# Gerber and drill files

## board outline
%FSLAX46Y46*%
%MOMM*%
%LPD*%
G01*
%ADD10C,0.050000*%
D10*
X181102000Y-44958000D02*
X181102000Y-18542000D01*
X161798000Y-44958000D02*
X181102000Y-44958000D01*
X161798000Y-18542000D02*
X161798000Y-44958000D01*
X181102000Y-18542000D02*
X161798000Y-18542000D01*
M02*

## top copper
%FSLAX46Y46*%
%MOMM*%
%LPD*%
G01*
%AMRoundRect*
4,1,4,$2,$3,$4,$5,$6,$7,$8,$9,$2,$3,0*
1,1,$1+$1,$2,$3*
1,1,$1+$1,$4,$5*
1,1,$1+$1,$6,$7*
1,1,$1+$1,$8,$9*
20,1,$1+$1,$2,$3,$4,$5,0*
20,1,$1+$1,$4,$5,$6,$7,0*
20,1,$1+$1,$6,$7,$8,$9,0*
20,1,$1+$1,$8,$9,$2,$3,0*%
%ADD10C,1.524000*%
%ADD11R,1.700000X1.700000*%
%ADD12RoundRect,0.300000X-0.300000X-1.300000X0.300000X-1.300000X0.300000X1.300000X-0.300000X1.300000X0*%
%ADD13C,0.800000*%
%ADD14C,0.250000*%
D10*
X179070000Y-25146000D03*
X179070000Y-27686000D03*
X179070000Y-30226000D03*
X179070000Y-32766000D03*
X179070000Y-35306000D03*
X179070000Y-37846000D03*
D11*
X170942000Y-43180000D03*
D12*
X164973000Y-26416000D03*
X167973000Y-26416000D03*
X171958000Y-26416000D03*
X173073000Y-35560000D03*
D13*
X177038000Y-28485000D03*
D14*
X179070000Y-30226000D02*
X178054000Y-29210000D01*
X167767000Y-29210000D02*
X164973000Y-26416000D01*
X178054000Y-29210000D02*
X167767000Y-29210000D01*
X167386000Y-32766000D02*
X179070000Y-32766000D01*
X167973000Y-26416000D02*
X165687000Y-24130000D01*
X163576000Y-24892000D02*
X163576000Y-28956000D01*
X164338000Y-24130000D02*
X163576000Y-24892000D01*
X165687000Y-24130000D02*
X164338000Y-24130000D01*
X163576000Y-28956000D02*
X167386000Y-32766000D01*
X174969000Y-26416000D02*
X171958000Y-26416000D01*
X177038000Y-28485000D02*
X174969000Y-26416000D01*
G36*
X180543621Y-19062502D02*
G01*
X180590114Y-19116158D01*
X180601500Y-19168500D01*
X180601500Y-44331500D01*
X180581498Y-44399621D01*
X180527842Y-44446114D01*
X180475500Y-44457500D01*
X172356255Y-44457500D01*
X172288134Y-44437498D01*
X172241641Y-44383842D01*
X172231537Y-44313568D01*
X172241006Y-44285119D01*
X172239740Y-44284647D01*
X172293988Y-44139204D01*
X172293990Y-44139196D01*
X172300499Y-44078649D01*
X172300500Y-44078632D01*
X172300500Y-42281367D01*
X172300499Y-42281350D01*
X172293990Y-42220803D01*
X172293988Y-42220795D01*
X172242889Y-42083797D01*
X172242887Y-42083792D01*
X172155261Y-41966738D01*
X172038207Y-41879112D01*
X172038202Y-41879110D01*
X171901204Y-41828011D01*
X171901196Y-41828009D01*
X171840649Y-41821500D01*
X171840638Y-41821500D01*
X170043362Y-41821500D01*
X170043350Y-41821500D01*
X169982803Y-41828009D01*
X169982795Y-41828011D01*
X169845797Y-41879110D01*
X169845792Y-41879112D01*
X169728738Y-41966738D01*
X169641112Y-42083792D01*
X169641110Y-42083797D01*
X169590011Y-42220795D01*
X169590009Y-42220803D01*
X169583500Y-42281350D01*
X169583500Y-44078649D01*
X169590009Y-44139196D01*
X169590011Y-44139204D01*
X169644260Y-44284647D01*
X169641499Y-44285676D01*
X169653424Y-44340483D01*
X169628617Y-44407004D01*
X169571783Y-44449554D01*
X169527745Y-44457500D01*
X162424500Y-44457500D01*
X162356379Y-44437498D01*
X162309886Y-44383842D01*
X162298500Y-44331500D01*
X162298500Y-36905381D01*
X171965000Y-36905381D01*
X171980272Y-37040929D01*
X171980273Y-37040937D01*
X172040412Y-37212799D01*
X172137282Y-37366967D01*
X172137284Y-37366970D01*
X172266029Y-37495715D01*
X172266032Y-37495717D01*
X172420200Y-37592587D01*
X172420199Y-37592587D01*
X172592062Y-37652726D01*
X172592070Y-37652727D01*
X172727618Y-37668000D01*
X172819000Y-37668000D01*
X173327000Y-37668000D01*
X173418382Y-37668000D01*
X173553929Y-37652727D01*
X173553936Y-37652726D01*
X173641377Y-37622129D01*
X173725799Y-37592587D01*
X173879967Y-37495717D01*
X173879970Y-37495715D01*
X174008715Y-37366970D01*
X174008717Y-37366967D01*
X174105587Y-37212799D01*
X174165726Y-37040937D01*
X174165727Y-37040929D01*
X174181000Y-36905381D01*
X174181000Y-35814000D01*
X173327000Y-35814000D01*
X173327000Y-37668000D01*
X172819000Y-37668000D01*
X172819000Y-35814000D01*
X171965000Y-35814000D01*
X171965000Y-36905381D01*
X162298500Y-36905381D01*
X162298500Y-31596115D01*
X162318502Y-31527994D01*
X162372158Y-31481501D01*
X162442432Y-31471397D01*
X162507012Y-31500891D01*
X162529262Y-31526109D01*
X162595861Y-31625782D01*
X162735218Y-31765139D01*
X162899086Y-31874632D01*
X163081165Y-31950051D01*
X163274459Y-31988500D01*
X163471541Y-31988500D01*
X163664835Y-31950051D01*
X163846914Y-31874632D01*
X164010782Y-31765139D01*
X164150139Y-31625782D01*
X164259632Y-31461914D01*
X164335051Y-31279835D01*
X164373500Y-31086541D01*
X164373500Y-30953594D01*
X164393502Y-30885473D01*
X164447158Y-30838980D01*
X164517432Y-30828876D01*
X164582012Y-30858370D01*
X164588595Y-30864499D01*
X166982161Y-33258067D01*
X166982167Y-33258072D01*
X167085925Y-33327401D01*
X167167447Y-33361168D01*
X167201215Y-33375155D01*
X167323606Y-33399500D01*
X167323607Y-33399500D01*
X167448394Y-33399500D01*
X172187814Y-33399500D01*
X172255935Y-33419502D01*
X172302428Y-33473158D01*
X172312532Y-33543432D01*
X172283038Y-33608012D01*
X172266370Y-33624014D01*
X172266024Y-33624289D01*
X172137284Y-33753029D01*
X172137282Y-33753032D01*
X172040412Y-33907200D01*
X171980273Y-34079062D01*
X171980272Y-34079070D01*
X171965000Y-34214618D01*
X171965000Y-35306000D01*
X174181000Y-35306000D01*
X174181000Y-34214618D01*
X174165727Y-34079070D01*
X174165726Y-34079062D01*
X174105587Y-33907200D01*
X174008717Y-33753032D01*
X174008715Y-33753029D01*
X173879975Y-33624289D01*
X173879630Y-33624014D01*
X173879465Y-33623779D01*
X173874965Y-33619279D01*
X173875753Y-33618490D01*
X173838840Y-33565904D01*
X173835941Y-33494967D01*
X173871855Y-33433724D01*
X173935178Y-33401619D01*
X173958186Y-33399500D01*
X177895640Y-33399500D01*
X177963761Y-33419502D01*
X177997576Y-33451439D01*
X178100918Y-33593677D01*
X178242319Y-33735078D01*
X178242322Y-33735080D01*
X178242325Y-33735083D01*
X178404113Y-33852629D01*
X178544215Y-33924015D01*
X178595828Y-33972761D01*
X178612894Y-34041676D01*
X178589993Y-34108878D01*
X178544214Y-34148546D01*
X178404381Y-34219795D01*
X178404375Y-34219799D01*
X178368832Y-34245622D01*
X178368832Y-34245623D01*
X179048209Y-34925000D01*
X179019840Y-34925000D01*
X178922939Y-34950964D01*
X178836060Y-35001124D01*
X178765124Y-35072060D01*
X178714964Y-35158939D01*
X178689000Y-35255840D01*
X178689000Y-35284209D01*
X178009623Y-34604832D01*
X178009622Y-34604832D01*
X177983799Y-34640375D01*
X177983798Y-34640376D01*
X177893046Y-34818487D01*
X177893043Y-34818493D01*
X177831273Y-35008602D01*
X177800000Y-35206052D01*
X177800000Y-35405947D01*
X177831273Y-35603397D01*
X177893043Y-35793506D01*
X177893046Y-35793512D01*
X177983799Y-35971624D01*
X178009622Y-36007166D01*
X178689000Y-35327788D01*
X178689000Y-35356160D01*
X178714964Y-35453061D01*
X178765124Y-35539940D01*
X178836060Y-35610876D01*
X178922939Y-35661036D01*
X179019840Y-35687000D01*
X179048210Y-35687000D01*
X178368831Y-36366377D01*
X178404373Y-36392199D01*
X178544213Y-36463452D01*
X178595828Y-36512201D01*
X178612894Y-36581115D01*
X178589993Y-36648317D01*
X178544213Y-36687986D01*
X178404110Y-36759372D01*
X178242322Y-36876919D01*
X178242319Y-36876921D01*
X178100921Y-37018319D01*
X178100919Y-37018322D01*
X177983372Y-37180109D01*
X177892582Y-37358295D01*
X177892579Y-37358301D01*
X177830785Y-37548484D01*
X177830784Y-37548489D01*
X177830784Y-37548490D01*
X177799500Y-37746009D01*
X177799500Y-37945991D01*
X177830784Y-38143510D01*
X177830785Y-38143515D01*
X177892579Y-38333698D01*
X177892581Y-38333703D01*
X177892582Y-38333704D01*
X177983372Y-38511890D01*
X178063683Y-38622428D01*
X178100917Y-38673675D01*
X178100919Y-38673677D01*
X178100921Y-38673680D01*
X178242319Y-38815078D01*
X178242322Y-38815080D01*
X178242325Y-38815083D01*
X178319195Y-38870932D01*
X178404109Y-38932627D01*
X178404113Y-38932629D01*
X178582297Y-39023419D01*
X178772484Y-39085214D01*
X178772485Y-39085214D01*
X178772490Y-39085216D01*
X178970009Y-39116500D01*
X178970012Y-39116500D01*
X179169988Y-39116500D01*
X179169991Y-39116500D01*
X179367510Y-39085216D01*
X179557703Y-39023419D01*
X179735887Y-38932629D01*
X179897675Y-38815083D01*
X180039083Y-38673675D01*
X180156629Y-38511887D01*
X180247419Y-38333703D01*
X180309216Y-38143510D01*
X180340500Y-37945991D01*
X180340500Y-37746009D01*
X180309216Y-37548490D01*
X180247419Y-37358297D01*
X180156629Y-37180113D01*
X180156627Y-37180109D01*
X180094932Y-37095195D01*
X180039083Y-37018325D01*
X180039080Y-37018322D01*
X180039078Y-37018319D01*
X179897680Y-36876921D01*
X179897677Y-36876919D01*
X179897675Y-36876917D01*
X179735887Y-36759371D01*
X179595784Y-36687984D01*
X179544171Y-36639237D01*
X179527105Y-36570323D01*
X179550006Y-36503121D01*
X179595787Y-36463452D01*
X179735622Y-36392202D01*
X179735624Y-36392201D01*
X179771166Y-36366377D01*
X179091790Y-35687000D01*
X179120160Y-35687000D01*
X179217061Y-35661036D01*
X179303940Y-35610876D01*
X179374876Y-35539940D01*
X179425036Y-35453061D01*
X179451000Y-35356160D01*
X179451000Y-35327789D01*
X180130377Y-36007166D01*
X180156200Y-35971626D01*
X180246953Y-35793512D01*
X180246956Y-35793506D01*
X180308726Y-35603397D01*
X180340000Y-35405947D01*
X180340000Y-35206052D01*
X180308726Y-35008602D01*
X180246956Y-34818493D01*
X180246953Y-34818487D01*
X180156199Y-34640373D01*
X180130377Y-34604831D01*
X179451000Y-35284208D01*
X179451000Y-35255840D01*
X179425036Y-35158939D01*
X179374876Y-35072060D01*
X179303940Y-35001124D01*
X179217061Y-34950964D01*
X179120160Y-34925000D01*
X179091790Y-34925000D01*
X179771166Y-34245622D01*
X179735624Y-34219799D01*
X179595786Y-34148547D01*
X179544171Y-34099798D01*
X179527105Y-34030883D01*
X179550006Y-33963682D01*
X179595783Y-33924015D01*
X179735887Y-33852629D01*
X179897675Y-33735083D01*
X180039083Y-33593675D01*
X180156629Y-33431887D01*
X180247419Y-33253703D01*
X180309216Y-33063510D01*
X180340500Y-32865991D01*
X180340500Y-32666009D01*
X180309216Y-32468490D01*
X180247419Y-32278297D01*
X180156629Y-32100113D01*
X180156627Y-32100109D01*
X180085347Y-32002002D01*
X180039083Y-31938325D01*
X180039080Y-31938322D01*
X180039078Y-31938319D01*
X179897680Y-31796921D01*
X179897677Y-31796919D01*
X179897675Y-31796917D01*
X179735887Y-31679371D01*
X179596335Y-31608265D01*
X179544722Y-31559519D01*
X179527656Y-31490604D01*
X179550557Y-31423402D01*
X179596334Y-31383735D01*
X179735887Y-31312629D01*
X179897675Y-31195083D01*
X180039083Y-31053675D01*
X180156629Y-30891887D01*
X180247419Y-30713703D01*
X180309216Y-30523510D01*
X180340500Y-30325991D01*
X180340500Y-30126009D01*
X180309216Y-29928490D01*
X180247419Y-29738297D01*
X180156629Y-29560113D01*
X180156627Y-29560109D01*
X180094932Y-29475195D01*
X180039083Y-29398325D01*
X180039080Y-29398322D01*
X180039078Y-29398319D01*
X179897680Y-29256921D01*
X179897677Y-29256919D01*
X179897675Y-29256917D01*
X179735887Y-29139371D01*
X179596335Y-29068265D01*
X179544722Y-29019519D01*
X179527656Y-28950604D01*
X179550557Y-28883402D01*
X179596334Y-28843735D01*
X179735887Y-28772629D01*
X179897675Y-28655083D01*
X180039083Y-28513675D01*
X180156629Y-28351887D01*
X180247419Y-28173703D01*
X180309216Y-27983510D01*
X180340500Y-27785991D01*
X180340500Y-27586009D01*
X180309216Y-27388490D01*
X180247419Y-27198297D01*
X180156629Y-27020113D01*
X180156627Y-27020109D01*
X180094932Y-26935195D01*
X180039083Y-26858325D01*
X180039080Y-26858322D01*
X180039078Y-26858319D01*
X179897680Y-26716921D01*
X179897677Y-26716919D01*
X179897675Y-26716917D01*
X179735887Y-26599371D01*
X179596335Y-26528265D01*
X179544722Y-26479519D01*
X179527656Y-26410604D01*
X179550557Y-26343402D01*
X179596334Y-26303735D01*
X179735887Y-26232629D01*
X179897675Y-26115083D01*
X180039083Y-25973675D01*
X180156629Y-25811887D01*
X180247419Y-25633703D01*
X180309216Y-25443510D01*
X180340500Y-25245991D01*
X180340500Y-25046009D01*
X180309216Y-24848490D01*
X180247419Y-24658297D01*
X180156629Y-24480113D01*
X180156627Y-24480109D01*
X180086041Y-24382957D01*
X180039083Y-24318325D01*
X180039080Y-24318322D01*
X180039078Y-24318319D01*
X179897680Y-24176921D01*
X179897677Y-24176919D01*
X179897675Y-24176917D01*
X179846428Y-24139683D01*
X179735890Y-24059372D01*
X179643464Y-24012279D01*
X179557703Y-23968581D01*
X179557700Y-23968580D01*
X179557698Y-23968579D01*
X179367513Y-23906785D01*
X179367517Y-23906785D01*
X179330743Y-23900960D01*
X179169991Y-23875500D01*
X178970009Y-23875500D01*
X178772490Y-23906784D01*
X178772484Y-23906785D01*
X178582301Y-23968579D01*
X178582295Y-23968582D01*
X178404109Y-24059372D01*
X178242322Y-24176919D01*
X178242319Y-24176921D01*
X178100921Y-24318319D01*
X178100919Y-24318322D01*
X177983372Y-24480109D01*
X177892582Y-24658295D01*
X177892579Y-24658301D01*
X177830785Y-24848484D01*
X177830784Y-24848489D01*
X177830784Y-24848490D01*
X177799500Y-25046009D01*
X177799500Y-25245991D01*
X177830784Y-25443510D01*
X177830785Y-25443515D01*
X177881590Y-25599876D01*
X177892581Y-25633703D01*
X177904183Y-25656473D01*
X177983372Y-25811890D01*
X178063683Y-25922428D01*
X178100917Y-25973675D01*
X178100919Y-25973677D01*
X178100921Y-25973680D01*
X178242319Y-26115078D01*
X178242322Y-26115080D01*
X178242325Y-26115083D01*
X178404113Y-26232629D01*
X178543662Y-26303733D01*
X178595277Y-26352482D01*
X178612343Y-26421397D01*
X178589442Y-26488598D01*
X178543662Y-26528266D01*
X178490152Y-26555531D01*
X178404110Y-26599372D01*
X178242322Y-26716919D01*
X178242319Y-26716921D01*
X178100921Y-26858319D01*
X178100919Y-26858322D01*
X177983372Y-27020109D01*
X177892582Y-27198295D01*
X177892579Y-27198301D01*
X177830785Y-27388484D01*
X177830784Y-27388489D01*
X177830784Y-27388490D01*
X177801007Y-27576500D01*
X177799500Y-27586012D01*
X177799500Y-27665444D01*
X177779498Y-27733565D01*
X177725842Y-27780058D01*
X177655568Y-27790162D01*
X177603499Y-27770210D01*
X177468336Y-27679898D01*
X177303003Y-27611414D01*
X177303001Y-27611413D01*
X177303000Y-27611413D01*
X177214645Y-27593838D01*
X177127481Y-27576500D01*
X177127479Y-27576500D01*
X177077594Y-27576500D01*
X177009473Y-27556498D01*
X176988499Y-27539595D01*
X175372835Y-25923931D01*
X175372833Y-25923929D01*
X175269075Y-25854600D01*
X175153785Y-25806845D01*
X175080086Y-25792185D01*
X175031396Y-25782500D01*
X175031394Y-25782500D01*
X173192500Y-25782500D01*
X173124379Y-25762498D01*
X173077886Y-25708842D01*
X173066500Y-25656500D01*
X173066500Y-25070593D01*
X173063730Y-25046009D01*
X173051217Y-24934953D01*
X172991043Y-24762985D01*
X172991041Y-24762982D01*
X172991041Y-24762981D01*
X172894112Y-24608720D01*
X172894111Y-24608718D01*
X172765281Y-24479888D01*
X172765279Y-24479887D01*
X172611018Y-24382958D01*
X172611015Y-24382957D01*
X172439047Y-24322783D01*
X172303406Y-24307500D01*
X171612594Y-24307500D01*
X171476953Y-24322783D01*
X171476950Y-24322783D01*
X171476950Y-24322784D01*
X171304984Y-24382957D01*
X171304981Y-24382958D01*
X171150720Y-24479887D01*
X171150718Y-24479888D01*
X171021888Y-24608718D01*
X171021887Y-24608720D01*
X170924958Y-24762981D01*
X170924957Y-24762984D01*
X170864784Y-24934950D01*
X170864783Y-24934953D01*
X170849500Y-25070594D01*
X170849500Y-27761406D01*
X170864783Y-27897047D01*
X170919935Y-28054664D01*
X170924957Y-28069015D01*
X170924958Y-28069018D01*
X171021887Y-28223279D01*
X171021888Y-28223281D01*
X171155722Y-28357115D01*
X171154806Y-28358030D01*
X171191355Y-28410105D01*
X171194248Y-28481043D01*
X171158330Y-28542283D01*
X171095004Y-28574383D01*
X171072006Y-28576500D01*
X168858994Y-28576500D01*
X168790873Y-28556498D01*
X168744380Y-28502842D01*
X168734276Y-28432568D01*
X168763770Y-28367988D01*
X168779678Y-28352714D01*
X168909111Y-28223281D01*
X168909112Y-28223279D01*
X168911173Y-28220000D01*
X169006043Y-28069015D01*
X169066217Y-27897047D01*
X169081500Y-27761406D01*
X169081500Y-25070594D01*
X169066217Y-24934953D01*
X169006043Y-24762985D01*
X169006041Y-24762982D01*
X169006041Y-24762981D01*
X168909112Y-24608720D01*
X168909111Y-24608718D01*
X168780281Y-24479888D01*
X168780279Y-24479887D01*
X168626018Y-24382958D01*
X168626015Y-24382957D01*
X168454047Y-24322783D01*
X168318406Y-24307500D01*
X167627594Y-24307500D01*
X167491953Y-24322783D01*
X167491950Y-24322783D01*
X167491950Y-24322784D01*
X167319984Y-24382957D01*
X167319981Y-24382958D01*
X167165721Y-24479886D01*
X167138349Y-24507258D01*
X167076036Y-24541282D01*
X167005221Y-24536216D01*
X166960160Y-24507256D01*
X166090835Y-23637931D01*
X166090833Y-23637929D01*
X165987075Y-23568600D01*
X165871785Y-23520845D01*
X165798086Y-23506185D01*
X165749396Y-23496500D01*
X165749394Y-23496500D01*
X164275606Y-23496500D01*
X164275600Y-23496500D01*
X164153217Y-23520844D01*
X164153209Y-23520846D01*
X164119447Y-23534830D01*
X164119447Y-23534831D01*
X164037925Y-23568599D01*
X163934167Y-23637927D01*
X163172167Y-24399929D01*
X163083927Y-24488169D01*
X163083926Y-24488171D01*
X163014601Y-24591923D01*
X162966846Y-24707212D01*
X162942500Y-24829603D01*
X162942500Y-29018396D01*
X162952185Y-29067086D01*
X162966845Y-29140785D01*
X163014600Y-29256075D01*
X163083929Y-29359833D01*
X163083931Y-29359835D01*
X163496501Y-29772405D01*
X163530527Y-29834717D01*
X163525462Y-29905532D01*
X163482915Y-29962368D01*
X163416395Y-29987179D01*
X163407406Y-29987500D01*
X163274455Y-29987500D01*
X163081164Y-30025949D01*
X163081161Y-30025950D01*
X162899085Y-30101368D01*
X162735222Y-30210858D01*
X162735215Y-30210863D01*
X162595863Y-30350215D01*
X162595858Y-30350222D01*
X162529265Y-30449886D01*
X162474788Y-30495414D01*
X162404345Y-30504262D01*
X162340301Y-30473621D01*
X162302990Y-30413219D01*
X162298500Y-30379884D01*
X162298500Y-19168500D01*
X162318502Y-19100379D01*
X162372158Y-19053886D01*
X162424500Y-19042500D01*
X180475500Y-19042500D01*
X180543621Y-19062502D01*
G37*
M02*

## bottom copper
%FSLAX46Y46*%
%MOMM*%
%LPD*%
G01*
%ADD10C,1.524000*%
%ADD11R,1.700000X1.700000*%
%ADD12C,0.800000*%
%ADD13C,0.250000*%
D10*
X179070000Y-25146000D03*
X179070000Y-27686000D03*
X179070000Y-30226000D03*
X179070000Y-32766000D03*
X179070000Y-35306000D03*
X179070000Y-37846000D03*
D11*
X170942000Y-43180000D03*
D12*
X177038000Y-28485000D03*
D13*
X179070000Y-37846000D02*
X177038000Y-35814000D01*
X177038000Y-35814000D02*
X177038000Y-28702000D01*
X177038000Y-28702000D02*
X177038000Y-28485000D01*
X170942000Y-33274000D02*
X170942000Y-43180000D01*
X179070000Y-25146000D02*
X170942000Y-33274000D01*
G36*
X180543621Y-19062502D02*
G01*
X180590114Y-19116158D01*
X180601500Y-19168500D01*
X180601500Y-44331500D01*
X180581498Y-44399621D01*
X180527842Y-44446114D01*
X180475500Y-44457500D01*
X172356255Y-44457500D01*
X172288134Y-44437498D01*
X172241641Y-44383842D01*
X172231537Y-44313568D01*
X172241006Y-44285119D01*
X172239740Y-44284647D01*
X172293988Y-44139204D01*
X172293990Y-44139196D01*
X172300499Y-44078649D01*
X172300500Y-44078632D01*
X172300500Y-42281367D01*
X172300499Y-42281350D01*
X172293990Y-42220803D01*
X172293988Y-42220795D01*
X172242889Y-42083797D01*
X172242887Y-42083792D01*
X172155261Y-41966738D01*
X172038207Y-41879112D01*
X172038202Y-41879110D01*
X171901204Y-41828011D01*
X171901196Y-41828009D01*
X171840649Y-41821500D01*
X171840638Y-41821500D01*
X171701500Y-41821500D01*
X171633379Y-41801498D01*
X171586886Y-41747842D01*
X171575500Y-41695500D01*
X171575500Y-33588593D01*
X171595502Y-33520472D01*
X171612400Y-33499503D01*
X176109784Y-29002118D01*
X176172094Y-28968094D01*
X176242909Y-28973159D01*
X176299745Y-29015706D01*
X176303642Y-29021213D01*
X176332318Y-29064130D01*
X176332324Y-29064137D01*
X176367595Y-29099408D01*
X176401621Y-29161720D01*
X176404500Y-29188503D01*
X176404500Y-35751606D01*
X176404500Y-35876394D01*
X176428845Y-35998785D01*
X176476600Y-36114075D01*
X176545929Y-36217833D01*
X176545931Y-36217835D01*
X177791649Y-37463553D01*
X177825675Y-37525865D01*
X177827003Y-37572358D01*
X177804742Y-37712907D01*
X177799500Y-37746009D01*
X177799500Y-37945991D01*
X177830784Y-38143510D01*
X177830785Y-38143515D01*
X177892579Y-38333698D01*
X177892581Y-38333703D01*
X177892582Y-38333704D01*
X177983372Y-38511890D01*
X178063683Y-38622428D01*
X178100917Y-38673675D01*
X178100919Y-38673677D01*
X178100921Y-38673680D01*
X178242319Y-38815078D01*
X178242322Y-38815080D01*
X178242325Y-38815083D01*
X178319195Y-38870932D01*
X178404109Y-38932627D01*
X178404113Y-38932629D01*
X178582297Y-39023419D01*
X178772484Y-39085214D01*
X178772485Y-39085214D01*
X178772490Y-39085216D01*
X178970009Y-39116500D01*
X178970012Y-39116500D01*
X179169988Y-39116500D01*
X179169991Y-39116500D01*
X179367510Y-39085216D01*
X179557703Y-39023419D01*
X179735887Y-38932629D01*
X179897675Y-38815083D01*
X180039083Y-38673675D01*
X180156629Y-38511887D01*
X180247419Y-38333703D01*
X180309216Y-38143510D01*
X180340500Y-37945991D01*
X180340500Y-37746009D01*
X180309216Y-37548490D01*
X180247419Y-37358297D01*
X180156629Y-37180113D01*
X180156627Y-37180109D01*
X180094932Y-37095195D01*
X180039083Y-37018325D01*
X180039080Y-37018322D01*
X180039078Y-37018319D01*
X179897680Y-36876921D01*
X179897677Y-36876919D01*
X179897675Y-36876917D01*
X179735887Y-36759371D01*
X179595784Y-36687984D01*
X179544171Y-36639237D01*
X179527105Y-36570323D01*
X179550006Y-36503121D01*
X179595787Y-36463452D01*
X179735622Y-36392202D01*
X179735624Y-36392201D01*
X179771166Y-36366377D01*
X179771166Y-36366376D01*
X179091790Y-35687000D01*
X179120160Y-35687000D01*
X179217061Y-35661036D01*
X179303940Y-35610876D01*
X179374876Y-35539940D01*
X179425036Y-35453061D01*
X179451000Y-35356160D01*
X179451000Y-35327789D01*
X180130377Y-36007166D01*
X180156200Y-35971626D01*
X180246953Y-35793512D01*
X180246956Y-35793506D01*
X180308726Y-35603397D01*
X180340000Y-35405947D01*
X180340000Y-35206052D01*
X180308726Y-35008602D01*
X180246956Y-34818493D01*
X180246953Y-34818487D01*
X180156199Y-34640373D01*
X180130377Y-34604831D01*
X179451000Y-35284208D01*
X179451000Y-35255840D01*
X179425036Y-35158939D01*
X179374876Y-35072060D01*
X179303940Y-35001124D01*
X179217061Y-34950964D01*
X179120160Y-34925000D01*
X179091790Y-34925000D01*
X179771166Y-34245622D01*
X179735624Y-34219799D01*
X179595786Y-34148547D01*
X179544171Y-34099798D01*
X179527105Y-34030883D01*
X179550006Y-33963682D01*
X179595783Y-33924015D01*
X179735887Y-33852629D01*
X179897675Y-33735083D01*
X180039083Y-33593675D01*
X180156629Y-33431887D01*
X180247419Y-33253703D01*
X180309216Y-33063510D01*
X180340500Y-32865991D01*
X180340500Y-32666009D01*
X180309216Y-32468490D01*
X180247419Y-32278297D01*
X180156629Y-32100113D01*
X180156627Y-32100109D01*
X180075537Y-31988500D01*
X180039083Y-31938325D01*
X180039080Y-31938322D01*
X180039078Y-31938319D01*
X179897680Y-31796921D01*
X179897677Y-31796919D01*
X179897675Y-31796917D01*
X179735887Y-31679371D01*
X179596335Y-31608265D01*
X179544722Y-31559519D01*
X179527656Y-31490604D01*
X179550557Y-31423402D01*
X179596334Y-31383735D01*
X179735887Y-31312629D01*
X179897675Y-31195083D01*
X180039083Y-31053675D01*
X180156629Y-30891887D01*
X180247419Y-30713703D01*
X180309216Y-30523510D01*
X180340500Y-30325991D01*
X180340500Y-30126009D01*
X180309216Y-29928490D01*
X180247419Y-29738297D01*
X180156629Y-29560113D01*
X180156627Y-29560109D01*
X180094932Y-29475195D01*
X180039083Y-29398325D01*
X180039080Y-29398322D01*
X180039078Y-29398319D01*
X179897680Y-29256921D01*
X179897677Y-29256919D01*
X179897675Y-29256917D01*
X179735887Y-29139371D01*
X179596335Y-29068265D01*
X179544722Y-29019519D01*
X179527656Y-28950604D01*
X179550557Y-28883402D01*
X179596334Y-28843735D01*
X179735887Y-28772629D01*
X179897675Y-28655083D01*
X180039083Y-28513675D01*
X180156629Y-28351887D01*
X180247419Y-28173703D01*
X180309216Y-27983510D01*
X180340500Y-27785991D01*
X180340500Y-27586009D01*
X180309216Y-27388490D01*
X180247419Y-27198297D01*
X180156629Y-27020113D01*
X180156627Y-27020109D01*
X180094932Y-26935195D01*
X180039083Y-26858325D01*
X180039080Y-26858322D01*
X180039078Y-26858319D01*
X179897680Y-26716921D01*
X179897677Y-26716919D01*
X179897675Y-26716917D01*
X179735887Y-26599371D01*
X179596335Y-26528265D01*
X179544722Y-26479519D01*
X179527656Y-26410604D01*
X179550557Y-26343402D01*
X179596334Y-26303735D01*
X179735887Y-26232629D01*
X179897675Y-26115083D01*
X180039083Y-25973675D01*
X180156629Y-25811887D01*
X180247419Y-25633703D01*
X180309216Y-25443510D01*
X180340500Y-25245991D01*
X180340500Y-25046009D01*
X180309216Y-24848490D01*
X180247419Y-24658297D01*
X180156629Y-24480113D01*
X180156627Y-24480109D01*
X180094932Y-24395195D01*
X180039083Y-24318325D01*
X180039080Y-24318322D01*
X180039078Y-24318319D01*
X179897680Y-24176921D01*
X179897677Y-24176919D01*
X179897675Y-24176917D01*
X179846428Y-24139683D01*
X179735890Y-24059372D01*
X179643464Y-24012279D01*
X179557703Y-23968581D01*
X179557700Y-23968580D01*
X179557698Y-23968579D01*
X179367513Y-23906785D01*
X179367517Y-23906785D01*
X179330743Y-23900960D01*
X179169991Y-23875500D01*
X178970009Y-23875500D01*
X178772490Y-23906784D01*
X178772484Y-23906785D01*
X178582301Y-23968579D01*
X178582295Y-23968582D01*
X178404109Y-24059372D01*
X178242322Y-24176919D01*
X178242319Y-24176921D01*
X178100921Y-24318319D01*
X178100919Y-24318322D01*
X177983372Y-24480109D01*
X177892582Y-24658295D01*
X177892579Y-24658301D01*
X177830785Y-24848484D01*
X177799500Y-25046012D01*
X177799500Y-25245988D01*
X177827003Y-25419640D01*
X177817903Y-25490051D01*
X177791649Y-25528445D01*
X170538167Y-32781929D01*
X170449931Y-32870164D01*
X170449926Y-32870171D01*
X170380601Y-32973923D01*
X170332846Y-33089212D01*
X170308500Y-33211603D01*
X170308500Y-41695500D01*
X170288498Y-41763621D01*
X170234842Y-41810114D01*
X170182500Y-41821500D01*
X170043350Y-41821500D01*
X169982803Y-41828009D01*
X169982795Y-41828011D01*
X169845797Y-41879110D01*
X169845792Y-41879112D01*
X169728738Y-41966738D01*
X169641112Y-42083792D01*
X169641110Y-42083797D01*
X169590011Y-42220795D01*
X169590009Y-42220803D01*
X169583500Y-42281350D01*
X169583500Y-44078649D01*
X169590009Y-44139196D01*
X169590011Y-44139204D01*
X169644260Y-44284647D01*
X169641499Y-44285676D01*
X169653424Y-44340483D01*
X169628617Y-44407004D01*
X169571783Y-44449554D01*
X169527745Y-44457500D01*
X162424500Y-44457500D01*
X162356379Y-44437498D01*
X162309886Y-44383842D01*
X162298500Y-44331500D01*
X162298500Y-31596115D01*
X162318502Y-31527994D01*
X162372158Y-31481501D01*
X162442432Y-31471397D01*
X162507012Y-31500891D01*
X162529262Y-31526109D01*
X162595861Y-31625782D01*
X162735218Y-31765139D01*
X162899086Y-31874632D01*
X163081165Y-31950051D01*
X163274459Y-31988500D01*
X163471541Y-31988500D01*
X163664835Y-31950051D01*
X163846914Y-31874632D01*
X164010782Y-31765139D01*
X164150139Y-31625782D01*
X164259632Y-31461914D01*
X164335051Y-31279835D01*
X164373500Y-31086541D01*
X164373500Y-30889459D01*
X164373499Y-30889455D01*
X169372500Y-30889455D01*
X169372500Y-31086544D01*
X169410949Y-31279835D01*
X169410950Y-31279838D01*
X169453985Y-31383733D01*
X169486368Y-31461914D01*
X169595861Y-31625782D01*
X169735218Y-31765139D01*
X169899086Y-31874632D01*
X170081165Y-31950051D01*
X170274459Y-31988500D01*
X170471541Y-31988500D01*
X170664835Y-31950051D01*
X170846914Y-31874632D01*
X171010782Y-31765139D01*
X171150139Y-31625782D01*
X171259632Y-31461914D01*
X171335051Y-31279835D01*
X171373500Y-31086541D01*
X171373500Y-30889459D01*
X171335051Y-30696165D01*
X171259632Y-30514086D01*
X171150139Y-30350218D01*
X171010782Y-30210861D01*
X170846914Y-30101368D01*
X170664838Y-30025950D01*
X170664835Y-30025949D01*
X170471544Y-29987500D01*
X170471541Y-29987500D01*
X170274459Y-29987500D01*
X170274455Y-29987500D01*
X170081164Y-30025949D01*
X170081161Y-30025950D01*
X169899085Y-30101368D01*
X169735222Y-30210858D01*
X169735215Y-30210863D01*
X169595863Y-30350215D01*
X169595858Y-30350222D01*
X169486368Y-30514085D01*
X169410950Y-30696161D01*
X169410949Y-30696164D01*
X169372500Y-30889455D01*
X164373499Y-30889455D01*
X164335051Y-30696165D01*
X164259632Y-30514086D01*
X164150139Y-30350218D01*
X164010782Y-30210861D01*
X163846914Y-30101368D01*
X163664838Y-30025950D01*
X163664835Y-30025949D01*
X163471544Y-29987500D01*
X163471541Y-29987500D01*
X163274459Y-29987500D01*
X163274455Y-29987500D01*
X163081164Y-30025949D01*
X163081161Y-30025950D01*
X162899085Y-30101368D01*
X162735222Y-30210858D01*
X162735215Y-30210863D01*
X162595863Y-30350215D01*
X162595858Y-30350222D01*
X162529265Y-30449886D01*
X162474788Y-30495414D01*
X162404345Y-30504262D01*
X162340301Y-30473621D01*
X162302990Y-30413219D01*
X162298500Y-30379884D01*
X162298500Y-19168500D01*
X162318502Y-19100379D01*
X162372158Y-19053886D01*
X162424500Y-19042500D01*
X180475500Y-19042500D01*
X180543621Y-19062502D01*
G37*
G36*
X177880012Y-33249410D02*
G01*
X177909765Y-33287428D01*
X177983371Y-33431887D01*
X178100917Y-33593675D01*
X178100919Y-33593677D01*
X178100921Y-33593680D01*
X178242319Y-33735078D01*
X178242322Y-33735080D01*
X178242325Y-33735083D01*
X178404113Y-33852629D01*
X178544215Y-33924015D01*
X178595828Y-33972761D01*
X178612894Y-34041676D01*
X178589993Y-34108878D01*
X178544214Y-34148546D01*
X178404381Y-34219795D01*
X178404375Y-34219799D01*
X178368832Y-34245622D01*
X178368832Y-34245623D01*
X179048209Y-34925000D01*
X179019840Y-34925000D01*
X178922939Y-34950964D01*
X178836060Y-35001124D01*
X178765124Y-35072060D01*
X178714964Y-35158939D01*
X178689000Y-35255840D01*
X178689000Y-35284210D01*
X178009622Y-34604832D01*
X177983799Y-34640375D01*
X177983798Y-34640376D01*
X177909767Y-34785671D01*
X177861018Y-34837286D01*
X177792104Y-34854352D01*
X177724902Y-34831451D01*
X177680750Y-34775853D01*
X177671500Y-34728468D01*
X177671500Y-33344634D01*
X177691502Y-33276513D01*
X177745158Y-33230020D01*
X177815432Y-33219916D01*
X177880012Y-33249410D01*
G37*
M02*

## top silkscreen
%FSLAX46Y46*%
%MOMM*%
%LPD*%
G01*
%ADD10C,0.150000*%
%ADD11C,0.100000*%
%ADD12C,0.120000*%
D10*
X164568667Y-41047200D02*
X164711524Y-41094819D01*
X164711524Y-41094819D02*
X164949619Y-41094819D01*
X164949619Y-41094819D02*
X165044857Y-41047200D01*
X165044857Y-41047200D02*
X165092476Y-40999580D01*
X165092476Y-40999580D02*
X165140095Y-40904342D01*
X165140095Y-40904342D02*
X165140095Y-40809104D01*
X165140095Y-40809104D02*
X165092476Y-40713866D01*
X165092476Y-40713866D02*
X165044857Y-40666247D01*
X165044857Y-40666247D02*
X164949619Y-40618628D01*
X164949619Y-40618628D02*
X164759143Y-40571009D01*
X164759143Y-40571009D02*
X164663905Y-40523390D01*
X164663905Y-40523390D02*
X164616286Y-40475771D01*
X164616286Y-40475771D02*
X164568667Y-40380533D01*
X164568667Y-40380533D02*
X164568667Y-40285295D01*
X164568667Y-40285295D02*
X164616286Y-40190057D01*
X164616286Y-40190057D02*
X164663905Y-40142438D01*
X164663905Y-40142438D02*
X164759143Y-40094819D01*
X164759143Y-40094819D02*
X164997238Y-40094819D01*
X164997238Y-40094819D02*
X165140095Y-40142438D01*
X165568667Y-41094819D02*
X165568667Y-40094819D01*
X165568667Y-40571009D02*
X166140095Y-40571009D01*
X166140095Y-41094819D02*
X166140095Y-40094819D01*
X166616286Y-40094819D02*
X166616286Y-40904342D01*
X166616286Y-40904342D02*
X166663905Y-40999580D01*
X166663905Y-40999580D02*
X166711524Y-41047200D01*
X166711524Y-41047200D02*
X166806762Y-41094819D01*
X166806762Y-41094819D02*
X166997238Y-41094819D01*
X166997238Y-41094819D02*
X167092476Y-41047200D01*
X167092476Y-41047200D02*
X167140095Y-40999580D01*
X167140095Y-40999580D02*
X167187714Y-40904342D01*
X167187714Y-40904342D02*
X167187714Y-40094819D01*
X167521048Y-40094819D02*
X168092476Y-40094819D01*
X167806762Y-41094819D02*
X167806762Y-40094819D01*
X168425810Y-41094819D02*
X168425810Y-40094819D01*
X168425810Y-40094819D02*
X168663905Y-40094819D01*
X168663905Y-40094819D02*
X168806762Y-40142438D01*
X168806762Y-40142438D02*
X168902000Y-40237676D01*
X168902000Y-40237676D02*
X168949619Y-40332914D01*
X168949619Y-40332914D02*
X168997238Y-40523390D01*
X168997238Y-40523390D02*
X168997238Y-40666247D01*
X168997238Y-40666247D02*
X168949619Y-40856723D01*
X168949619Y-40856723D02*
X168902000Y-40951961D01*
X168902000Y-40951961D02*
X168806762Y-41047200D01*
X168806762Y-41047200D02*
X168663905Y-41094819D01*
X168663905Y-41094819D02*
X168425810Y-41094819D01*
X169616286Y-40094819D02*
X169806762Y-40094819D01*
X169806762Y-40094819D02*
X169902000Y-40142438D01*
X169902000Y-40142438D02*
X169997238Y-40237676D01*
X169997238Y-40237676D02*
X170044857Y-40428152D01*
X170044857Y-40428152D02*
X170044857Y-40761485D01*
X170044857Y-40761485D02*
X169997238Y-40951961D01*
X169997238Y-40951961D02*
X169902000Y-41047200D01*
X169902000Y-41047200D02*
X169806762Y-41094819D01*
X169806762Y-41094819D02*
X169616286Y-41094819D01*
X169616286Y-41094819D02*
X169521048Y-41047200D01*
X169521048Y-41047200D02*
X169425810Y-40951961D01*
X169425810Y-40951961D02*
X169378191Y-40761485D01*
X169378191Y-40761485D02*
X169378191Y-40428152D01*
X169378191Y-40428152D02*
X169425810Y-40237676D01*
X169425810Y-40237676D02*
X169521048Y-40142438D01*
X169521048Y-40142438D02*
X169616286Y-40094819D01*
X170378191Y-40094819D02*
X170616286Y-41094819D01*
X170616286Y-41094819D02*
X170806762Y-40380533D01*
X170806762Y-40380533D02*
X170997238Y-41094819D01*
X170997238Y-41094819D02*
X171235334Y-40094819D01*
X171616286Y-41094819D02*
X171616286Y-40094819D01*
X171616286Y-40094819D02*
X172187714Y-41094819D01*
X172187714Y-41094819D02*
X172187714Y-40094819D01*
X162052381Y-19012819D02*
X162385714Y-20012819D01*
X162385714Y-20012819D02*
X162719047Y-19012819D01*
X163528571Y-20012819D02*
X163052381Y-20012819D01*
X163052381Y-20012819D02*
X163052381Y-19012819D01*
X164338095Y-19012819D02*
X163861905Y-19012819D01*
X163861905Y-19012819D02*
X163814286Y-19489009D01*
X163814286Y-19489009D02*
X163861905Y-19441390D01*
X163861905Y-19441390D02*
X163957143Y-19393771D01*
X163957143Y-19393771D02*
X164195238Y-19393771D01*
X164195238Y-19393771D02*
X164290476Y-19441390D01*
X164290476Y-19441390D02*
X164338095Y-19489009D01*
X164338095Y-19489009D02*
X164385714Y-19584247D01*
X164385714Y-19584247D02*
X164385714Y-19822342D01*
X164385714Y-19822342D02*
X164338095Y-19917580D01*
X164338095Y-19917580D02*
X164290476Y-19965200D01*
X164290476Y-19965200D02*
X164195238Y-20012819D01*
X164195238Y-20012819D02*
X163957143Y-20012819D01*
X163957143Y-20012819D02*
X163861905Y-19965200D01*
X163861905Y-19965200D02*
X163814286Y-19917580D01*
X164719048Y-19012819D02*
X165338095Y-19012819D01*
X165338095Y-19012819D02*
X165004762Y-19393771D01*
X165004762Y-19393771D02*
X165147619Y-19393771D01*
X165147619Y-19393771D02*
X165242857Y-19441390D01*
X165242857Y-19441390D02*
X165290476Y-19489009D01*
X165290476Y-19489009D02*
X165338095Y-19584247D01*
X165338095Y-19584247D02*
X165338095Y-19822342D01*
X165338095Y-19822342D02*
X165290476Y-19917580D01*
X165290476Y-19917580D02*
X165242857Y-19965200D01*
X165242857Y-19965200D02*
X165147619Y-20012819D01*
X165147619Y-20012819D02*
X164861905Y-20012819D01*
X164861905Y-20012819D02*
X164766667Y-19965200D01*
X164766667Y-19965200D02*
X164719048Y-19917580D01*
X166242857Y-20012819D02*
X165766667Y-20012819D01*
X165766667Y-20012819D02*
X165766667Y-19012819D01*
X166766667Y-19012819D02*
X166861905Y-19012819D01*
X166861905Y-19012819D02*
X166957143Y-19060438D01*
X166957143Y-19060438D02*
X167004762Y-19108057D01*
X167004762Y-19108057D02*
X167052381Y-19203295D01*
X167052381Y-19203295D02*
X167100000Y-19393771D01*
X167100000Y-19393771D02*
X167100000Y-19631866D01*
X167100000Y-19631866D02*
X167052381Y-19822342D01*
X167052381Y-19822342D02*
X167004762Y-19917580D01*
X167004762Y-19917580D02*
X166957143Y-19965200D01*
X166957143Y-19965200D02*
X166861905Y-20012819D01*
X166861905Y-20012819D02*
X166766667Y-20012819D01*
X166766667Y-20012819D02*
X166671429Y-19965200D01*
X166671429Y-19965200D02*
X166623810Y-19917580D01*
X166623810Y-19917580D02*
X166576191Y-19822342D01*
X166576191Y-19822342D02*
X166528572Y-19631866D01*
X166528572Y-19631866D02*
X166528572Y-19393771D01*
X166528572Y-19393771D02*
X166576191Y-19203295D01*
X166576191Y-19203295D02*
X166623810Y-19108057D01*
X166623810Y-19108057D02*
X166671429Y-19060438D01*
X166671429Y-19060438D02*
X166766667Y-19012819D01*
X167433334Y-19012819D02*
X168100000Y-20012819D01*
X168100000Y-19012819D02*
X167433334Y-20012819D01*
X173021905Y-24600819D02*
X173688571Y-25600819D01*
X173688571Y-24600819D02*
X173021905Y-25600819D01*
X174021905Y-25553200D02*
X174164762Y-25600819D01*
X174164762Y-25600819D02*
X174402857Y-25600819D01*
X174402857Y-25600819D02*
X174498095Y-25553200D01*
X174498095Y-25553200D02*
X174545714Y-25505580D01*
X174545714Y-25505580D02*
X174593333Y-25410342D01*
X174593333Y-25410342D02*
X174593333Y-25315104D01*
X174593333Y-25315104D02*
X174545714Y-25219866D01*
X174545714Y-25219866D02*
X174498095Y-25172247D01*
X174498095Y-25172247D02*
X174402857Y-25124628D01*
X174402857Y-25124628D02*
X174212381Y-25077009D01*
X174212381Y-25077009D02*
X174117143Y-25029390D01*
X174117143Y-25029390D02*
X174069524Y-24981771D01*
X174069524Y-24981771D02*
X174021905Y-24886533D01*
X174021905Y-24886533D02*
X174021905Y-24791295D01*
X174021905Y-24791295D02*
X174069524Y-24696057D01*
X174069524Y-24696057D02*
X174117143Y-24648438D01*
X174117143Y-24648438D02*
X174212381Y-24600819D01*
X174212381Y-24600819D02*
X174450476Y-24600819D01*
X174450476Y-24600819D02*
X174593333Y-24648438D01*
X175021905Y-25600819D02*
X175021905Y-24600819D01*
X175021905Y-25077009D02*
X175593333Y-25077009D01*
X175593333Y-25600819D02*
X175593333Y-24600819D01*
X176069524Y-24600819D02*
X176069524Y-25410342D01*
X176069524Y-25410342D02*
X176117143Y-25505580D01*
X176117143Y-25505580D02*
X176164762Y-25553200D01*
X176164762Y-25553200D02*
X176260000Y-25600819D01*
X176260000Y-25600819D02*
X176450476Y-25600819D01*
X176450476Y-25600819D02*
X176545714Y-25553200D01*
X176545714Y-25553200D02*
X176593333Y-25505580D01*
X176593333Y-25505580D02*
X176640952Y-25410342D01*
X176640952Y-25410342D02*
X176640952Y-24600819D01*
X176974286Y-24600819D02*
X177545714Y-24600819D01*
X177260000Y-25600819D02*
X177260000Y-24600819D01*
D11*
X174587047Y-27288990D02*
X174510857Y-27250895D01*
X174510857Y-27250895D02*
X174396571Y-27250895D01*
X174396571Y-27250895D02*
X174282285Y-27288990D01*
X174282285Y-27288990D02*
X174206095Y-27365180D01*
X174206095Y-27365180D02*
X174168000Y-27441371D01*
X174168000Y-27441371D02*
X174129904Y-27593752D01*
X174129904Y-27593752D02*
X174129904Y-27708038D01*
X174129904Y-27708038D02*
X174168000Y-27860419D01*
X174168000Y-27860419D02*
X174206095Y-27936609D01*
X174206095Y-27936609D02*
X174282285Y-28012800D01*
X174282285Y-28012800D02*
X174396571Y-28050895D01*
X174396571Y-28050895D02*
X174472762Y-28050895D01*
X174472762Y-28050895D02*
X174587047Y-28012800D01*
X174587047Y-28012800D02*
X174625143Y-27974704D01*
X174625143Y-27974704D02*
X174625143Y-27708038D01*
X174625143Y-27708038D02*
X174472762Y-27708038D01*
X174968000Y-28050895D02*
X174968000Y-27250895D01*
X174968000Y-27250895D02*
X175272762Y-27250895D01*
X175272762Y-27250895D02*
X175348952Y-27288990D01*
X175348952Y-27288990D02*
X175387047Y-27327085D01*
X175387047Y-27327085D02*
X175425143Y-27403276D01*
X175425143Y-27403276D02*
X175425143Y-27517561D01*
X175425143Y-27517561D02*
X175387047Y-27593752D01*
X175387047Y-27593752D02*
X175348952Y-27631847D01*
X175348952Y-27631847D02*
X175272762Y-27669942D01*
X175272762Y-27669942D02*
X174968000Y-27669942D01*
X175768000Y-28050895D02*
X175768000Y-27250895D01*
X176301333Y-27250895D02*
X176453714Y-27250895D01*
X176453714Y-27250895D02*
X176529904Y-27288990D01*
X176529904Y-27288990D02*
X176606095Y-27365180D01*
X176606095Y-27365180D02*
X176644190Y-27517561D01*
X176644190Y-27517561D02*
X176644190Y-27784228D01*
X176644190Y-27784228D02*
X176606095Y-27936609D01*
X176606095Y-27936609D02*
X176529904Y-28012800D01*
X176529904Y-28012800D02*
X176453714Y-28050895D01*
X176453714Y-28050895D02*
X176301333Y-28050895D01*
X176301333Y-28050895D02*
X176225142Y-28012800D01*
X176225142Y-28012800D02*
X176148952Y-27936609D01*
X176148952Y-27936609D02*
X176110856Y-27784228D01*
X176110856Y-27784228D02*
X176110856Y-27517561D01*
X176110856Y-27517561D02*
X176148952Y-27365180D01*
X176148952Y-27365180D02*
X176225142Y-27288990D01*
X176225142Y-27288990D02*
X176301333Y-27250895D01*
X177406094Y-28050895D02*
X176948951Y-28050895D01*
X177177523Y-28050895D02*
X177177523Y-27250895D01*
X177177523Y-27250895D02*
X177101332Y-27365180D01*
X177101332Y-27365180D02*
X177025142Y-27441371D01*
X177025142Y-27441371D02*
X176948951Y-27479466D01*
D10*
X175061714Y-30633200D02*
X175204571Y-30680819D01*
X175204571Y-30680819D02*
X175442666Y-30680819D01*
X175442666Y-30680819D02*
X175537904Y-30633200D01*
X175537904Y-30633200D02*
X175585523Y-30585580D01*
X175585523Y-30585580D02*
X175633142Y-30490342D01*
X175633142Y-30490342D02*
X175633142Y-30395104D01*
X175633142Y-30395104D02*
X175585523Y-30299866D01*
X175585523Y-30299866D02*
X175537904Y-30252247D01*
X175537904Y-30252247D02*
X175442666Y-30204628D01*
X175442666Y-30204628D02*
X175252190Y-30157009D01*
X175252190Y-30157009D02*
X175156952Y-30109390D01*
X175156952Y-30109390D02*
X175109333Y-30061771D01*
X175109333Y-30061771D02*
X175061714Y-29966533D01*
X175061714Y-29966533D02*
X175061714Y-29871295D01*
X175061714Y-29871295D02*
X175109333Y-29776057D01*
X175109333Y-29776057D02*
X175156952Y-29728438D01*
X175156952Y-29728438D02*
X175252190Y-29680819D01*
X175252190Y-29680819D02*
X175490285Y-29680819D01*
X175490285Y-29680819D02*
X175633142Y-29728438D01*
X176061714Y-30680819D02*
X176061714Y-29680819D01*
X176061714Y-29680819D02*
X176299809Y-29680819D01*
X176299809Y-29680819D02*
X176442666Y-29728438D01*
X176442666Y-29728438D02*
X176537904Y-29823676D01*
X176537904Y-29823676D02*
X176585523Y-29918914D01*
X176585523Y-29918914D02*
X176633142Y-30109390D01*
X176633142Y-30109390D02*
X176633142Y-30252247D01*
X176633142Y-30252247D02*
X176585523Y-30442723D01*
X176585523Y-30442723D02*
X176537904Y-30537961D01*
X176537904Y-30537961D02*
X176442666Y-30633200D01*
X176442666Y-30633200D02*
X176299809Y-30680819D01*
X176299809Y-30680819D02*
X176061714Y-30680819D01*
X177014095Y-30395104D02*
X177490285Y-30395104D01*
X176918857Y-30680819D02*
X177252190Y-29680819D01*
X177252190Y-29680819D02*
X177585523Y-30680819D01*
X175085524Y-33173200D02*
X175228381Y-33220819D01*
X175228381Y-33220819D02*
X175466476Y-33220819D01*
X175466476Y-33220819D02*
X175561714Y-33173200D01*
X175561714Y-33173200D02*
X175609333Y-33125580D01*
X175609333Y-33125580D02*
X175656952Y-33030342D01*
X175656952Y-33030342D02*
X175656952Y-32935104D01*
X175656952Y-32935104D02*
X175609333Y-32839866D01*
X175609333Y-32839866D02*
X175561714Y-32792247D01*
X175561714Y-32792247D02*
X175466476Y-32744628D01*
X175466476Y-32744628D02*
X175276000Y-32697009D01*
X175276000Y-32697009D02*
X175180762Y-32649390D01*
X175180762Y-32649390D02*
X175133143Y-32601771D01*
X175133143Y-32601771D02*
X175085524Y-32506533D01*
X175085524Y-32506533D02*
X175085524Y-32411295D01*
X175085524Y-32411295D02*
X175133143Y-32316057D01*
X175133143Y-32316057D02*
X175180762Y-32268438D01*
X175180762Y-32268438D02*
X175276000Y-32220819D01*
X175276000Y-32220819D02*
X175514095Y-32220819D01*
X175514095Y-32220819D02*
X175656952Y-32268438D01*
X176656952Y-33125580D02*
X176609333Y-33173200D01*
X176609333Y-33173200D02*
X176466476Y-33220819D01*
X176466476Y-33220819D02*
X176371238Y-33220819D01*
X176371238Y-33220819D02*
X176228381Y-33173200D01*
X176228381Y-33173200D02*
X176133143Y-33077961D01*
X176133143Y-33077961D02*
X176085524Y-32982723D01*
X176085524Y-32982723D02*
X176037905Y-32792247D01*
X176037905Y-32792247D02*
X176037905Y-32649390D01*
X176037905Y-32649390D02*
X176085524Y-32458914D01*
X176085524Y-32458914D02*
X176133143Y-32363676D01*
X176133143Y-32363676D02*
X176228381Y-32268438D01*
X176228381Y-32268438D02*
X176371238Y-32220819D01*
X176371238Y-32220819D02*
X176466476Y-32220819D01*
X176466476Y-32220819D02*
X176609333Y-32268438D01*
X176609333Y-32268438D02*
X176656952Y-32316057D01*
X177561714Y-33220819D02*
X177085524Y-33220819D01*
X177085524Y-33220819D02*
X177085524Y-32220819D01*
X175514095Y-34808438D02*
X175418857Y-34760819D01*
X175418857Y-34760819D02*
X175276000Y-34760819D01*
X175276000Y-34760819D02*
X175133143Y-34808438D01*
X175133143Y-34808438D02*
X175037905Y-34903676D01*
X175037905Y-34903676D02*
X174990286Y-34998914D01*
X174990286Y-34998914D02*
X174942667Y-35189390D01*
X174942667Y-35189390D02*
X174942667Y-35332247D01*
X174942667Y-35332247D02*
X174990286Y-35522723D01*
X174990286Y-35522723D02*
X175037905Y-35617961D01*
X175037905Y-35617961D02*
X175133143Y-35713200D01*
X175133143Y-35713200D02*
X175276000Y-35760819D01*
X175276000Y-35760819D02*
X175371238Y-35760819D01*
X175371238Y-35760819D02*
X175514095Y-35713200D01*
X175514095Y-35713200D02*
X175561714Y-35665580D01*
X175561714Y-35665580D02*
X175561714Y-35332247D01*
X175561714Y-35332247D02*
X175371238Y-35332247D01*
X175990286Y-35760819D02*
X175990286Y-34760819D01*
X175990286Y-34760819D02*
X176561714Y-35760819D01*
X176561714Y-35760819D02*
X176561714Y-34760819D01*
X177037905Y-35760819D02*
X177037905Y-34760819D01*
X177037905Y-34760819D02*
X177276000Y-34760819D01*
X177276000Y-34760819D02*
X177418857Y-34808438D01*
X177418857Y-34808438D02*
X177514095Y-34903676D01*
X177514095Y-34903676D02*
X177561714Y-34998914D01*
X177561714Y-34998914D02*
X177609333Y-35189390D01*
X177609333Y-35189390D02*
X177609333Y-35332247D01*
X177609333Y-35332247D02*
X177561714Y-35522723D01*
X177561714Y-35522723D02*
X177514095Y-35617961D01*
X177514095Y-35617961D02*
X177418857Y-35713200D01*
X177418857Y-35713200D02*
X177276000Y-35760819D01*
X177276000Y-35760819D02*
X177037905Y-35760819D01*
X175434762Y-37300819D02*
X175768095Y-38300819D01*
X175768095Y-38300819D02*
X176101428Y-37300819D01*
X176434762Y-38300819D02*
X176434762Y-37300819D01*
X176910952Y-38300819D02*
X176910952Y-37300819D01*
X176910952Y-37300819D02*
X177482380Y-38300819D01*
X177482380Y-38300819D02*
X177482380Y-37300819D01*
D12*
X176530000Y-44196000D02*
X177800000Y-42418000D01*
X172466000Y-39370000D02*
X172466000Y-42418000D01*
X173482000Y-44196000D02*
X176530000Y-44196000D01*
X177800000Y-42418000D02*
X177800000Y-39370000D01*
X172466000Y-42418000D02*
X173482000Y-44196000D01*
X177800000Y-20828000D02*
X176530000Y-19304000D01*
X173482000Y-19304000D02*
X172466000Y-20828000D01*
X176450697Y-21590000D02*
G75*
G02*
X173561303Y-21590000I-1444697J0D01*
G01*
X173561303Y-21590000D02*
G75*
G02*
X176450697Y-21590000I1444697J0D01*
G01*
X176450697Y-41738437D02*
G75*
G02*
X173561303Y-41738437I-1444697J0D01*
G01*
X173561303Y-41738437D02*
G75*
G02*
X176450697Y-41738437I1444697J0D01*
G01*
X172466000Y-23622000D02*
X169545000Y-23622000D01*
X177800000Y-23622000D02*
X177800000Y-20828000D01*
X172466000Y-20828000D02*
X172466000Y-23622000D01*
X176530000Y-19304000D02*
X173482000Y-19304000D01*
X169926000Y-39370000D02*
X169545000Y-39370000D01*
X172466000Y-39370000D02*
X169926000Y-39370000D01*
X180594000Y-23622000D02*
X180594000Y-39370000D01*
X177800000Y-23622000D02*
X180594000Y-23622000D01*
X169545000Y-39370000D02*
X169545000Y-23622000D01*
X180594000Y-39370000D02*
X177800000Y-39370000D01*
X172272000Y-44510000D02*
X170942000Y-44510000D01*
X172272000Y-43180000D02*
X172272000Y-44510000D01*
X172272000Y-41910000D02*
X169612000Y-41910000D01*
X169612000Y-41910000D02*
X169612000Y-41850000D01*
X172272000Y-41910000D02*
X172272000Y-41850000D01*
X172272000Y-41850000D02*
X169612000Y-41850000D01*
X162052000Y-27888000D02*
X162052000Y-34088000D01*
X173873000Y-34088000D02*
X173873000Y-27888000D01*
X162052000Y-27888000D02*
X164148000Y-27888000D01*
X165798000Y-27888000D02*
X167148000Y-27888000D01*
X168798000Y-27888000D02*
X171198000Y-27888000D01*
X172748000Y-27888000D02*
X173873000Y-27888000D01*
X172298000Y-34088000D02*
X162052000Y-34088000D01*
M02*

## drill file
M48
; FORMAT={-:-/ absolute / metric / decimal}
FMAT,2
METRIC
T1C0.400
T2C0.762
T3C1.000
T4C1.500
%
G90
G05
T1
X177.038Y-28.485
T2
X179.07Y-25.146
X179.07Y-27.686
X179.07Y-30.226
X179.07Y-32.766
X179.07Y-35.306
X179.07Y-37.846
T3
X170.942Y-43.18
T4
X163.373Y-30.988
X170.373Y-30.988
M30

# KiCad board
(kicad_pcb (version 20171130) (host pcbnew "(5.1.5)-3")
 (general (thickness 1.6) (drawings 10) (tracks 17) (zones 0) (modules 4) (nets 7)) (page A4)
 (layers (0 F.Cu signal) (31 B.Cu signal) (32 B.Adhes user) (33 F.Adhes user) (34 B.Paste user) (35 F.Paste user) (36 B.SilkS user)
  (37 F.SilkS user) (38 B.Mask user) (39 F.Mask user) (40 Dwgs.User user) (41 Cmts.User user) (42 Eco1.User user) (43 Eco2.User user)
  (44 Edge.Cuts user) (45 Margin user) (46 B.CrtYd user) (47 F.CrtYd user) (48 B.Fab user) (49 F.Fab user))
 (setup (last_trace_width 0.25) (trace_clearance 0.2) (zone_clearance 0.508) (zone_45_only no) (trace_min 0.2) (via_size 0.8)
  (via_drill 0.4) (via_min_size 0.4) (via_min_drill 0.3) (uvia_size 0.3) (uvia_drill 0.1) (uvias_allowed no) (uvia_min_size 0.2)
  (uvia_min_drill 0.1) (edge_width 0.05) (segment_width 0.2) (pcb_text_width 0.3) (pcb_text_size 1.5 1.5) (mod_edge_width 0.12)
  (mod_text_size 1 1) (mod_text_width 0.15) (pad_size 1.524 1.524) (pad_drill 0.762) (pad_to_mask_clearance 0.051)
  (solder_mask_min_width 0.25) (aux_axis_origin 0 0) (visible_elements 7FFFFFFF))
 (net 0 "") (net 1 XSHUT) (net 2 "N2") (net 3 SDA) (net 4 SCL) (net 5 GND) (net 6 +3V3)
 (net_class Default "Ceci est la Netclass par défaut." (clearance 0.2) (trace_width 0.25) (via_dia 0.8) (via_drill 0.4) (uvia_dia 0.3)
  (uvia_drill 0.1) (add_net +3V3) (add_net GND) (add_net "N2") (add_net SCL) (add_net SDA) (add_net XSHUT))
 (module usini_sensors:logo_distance (layer B.Cu) (at 165.354 21.336 90)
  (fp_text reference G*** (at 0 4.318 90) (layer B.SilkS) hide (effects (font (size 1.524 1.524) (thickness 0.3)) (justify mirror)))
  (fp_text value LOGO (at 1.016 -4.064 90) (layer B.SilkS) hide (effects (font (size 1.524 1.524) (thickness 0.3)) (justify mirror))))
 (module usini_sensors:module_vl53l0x (layer F.Cu) (at 179.07 22.606 180)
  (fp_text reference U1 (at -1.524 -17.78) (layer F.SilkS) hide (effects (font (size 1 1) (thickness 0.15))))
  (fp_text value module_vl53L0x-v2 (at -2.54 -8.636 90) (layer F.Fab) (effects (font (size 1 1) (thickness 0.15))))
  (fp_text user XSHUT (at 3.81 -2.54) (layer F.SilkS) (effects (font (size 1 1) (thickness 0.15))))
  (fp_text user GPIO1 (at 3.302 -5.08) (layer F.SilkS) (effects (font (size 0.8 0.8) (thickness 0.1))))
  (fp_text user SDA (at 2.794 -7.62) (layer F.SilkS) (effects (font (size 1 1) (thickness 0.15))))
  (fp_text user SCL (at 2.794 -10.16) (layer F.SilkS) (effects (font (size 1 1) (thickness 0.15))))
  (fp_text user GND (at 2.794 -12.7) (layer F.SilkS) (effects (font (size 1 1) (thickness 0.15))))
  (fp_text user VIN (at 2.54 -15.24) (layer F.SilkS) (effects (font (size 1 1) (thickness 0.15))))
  (fp_line (start 2.54 -21.59) (end 1.27 -19.812) (layer F.SilkS) (width 0.12))
  (fp_line (start 6.604 -16.764) (end 6.604 -19.812) (layer F.SilkS) (width 0.12))
  (fp_line (start 5.588 -21.59) (end 2.54 -21.59) (layer F.SilkS) (width 0.12))
  (fp_line (start 1.27 -19.812) (end 1.27 -16.764) (layer F.SilkS) (width 0.12))
  (fp_line (start 6.604 -19.812) (end 5.588 -21.59) (layer F.SilkS) (width 0.12))
  (fp_line (start 1.27 1.778) (end 2.54 3.302) (layer F.SilkS) (width 0.12))
  (fp_line (start 5.588 3.302) (end 6.604 1.778) (layer F.SilkS) (width 0.12))
  (fp_circle (center 4.064 1.016) (end 4.572 2.368437) (layer F.SilkS) (width 0.12))
  (fp_circle (center 4.064 -19.132437) (end 4.572 -17.78) (layer F.SilkS) (width 0.12))
  (fp_line (start 6.604 -1.016) (end 9.525 -1.016) (layer F.SilkS) (width 0.12))
  (fp_line (start 1.27 -1.016) (end 1.27 1.778) (layer F.SilkS) (width 0.12))
  (fp_line (start 6.604 1.778) (end 6.604 -1.016) (layer F.SilkS) (width 0.12))
  (fp_line (start 2.54 3.302) (end 5.588 3.302) (layer F.SilkS) (width 0.12))
  (fp_line (start 9.144 -16.764) (end 9.525 -16.764) (layer F.SilkS) (width 0.12))
  (fp_line (start 6.604 -16.764) (end 9.144 -16.764) (layer F.SilkS) (width 0.12))
  (fp_line (start -1.524 -1.016) (end -1.524 -16.764) (layer F.SilkS) (width 0.12))
  (fp_line (start 1.27 -1.016) (end -1.524 -1.016) (layer F.SilkS) (width 0.12))
  (fp_line (start 9.525 -16.764) (end 9.525 -1.016) (layer F.SilkS) (width 0.12))
  (fp_line (start -1.524 -16.764) (end 1.27 -16.764) (layer F.SilkS) (width 0.12))
  (pad 6 thru_hole circle (at 0 -2.54 180) (size 1.524 1.524) (drill 0.762) (layers *.Cu *.Mask) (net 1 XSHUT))
  (pad 5 thru_hole circle (at 0 -5.08 180) (size 1.524 1.524) (drill 0.762) (layers *.Cu *.Mask) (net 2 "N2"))
  (pad 4 thru_hole circle (at 0 -7.62 180) (size 1.524 1.524) (drill 0.762) (layers *.Cu *.Mask) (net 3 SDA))
  (pad 3 thru_hole circle (at 0 -10.16 180) (size 1.524 1.524) (drill 0.762) (layers *.Cu *.Mask) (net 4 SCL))
  (pad 2 thru_hole circle (at 0 -12.7 180) (size 1.524 1.524) (drill 0.762) (layers *.Cu *.Mask) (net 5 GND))
  (pad 1 thru_hole circle (at 0 -15.24 180) (size 1.524 1.524) (drill 0.762) (layers *.Cu *.Mask) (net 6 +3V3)))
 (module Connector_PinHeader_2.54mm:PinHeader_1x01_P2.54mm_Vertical (layer F.Cu) (at 170.942 43.18 180)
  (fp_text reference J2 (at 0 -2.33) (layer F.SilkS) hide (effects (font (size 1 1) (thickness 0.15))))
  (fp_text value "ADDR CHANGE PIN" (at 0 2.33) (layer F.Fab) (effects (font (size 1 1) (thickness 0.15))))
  (fp_line (start -1.33 -1.33) (end 0 -1.33) (layer F.SilkS) (width 0.12))
  (fp_line (start -1.33 0) (end -1.33 -1.33) (layer F.SilkS) (width 0.12))
  (fp_line (start -1.33 1.27) (end 1.33 1.27) (layer F.SilkS) (width 0.12))
  (fp_line (start 1.33 1.27) (end 1.33 1.33) (layer F.SilkS) (width 0.12))
  (fp_line (start -1.33 1.27) (end -1.33 1.33) (layer F.SilkS) (width 0.12))
  (fp_line (start -1.33 1.33) (end 1.33 1.33) (layer F.SilkS) (width 0.12))
  (pad 1 thru_hole rect (at 0 0 180) (size 1.7 1.7) (drill 1) (layers *.Cu *.Mask) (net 1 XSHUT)))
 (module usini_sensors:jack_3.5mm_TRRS (layer F.Cu) (at 168.148 30.988)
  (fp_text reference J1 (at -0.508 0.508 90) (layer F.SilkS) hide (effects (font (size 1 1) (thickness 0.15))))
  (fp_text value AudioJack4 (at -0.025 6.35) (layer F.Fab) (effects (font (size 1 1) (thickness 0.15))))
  (fp_line (start -6.096 -3.1) (end -6.096 3.1) (layer F.SilkS) (width 0.12))
  (fp_line (start 5.725 3.1) (end 5.725 -3.1) (layer F.SilkS) (width 0.12))
  (fp_line (start -6.096 -3.1) (end -4 -3.1) (layer F.SilkS) (width 0.12))
  (fp_line (start -2.35 -3.1) (end -1 -3.1) (layer F.SilkS) (width 0.12))
  (fp_line (start 0.65 -3.1) (end 3.05 -3.1) (layer F.SilkS) (width 0.12))
  (fp_line (start 4.6 -3.1) (end 5.725 -3.1) (layer F.SilkS) (width 0.12))
  (fp_line (start 4.15 3.1) (end -6.096 3.1) (layer F.SilkS) (width 0.12))
  (pad "" np_thru_hole circle (at 2.225 0) (size 1.5 1.5) (drill 1.5) (layers *.Cu *.Mask))
  (pad "" np_thru_hole circle (at -4.775 0) (size 1.5 1.5) (drill 1.5) (layers *.Cu *.Mask))
  (pad R2 smd roundrect (at -3.175 -4.572) (size 1.2 3.2) (layers F.Cu F.Paste F.Mask) (roundrect_rratio 0.25) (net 3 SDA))
  (pad R1 smd roundrect (at -0.175 -4.572) (size 1.2 3.2) (layers F.Cu F.Paste F.Mask) (roundrect_rratio 0.25) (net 4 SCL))
  (pad T smd roundrect (at 3.81 -4.572) (size 1.2 3.2) (layers F.Cu F.Paste F.Mask) (roundrect_rratio 0.25) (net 6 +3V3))
  (pad S smd roundrect (at 4.925 4.572) (size 1.2 3.2) (layers F.Cu F.Paste F.Mask) (roundrect_rratio 0.25) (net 5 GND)))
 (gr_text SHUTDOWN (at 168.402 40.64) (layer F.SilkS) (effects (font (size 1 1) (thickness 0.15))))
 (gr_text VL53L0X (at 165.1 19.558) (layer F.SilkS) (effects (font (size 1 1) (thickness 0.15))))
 (gr_line (start 181.102 44.958) (end 181.102 18.542) (layer Edge.Cuts) (width 0.05))
 (gr_line (start 161.798 44.958) (end 181.102 44.958) (layer Edge.Cuts) (width 0.05))
 (gr_line (start 161.798 18.542) (end 161.798 44.958) (layer Edge.Cuts) (width 0.05))
 (gr_line (start 181.102 18.542) (end 161.798 18.542) (layer Edge.Cuts) (width 0.05))
 (segment (start 179.07 30.226) (end 178.054 29.21) (width 0.25) (layer F.Cu) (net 3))
 (segment (start 167.767 29.21) (end 164.973 26.416) (width 0.25) (layer F.Cu) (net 3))
 (segment (start 178.054 29.21) (end 167.767 29.21) (width 0.25) (layer F.Cu) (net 3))
 (segment (start 167.386 32.766) (end 179.07 32.766) (width 0.25) (layer F.Cu) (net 4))
 (segment (start 167.973 26.416) (end 165.687 24.13) (width 0.25) (layer F.Cu) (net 4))
 (segment (start 163.576 24.892) (end 163.576 28.956) (width 0.25) (layer F.Cu) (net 4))
 (segment (start 164.338 24.13) (end 163.576 24.892) (width 0.25) (layer F.Cu) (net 4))
 (segment (start 165.687 24.13) (end 164.338 24.13) (width 0.25) (layer F.Cu) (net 4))
 (segment (start 163.576 28.956) (end 167.386 32.766) (width 0.25) (layer F.Cu) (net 4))
 (segment (start 179.07 37.846) (end 177.038 35.814) (width 0.25) (layer B.Cu) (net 6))
 (segment (start 177.038 35.814) (end 177.038 28.702) (width 0.25) (layer B.Cu) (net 6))
 (via (at 177.038 28.485) (size 0.8) (drill 0.4) (layers F.Cu B.Cu) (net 6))
 (segment (start 177.038 28.702) (end 177.038 28.485) (width 0.25) (layer B.Cu) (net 6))
 (segment (start 174.969 26.416) (end 171.958 26.416) (width 0.25) (layer F.Cu) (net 6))
 (segment (start 177.038 28.485) (end 174.969 26.416) (width 0.25) (layer F.Cu) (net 6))
 (segment (start 170.942 33.274) (end 170.942 43.18) (width 0.25) (layer B.Cu) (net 1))
 (segment (start 179.07 25.146) (end 170.942 33.274) (width 0.25) (layer B.Cu) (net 1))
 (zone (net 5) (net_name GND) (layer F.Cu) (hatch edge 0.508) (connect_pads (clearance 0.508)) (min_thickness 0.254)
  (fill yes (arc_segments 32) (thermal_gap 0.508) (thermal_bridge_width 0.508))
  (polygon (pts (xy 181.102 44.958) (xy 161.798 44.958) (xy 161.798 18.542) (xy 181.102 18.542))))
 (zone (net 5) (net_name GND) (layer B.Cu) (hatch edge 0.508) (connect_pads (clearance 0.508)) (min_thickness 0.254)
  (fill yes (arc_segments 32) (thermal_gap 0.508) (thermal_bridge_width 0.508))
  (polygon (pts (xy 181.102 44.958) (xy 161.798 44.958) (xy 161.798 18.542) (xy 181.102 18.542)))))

